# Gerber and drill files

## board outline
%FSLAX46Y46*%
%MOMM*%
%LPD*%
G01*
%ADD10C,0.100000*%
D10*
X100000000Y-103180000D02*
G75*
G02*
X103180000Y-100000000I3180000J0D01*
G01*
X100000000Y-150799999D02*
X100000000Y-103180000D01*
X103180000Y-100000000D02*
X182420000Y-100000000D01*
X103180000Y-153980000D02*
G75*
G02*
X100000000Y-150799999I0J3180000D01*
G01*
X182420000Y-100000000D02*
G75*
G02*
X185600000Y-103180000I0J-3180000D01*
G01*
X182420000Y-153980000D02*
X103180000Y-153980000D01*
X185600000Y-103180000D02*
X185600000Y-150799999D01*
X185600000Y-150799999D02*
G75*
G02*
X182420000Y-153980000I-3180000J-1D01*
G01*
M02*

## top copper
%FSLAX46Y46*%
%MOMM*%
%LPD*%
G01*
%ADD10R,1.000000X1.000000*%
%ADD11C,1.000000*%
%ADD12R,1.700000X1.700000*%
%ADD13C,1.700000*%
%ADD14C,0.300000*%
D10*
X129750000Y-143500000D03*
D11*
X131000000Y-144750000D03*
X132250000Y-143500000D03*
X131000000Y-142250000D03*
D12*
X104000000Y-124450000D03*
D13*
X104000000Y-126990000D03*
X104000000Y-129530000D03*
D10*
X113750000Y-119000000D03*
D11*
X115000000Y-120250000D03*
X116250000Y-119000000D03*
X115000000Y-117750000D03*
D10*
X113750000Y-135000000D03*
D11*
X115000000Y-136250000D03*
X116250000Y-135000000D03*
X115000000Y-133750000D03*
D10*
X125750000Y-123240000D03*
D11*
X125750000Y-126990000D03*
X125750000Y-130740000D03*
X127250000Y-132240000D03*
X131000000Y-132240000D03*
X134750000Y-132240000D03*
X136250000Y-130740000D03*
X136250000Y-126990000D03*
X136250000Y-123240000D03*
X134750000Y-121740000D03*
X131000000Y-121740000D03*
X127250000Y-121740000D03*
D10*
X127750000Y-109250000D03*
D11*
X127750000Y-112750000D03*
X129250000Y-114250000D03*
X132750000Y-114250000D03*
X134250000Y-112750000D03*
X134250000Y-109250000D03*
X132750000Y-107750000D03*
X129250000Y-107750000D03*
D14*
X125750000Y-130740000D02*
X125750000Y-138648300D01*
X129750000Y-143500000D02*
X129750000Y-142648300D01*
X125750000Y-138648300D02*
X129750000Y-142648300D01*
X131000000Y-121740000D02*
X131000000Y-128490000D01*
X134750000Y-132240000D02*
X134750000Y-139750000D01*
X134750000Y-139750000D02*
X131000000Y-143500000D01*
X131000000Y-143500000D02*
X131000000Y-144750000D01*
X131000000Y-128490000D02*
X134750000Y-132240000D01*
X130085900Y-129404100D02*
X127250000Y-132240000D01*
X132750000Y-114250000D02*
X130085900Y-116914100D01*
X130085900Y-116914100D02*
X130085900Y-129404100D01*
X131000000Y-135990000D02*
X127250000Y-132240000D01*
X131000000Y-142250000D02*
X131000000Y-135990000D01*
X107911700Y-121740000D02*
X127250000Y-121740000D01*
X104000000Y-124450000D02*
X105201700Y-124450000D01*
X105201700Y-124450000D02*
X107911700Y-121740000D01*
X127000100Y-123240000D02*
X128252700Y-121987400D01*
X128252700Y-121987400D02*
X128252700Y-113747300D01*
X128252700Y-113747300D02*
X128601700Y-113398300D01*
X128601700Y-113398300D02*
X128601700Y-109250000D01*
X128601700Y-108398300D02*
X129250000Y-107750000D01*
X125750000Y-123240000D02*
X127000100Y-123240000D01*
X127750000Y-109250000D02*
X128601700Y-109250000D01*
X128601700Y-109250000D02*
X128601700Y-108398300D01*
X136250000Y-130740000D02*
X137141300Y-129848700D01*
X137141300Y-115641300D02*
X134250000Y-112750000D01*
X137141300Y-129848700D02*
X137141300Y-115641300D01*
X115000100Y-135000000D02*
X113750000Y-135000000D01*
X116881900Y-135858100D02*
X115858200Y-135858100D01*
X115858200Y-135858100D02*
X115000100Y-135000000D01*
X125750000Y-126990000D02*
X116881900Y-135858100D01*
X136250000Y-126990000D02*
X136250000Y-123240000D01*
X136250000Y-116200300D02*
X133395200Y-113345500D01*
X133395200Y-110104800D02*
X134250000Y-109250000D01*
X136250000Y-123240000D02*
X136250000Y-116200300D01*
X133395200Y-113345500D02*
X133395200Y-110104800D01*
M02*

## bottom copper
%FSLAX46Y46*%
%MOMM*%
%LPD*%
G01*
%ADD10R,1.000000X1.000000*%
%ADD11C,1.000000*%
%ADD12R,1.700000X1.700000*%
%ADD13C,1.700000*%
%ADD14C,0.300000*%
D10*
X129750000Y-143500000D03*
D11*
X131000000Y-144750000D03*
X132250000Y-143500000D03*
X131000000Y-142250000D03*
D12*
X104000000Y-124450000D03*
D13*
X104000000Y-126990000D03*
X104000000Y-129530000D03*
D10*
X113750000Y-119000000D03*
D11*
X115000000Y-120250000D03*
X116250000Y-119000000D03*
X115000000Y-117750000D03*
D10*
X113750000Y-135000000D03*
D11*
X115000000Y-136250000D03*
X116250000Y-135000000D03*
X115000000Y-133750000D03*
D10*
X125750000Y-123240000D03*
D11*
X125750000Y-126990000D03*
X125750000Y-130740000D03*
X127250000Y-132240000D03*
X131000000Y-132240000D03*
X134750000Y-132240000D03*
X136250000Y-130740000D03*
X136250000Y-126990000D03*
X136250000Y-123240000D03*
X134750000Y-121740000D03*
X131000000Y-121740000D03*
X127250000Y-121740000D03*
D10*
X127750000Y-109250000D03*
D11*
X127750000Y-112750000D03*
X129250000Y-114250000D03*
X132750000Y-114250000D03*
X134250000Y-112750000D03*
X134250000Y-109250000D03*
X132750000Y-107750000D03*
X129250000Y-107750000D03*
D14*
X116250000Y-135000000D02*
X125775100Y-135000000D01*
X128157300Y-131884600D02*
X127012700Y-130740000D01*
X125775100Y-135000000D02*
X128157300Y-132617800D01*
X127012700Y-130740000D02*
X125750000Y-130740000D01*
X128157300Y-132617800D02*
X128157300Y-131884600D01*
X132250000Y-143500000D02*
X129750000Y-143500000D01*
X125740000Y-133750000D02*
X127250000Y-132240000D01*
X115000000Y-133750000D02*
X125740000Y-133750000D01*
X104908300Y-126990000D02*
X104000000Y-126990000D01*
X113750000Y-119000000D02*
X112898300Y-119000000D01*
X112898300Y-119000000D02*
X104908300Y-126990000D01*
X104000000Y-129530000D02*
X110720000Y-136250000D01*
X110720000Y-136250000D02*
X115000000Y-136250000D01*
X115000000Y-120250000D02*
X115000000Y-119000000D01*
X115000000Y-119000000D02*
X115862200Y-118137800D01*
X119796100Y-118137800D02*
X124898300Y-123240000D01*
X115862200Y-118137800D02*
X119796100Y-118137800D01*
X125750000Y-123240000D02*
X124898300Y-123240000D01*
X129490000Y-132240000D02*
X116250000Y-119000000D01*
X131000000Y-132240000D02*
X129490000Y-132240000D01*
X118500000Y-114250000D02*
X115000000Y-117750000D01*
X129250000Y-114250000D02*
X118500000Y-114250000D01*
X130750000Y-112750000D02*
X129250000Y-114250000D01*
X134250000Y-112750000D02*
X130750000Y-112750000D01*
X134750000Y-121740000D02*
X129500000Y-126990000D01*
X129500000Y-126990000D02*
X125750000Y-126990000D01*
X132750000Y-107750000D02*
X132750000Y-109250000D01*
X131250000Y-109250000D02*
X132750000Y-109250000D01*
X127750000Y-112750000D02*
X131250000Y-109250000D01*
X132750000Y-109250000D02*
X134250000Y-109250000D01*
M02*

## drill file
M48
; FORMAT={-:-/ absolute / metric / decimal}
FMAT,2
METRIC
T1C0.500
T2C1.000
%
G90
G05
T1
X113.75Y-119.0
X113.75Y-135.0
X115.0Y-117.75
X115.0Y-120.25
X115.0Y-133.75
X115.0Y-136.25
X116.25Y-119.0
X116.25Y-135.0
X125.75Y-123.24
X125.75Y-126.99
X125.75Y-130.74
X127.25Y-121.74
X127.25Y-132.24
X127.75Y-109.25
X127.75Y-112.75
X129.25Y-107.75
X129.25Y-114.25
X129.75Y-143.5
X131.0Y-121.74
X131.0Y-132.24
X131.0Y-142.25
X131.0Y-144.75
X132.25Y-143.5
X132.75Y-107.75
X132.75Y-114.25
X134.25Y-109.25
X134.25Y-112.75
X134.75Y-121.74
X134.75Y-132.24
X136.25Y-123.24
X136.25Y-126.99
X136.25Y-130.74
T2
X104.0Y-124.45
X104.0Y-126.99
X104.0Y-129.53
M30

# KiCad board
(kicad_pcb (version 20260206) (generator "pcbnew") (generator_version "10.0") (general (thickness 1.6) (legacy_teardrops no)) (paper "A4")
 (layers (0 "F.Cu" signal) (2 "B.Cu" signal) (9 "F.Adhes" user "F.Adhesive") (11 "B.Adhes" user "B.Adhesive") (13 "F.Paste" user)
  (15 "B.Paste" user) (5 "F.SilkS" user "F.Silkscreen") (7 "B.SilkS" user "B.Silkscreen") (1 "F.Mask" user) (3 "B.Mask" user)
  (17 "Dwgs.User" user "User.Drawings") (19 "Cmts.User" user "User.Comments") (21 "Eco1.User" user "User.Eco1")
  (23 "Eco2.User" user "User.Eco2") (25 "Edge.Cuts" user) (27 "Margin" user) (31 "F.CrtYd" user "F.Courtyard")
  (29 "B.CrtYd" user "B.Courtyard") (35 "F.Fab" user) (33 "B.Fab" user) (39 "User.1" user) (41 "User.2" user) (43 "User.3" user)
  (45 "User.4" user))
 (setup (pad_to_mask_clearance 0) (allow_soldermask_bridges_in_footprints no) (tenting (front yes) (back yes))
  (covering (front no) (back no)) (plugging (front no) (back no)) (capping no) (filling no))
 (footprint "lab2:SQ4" (layer "F.Cu") (at 131 143.5)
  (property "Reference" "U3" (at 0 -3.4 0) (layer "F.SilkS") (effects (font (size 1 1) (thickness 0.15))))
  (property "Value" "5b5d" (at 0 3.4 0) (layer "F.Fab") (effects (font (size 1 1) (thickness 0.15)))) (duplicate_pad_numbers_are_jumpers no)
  (pad "1" thru_hole rect (at -1.25 0) (size 1 1) (drill 0.5) (layers "*.Cu" "*.Mask") (remove_unused_layers no) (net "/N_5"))
  (pad "2" thru_hole circle (at 0 1.25) (size 1 1) (drill 0.5) (layers "*.Cu" "*.Mask") (remove_unused_layers no) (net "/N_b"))
  (pad "3" thru_hole circle (at 1.25 0) (size 1 1) (drill 0.5) (layers "*.Cu" "*.Mask") (remove_unused_layers no) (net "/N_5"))
  (pad "4" thru_hole circle (at 0 -1.25) (size 1 1) (drill 0.5) (layers "*.Cu" "*.Mask") (remove_unused_layers no) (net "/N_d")))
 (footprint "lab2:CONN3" (layer "F.Cu") (at 104 126.99)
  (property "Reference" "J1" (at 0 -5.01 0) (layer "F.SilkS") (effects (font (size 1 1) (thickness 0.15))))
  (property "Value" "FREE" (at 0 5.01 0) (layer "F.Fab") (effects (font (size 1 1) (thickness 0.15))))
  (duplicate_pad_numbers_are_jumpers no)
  (pad "1" thru_hole rect (at 0 -2.54) (size 1.7 1.7) (drill 1) (layers "*.Cu" "*.Mask") (remove_unused_layers no) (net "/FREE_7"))
  (pad "2" thru_hole circle (at 0 0) (size 1.7 1.7) (drill 1) (layers "*.Cu" "*.Mask") (remove_unused_layers no) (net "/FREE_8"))
  (pad "3" thru_hole circle (at 0 2.54) (size 1.7 1.7) (drill 1) (layers "*.Cu" "*.Mask") (remove_unused_layers no) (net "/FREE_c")))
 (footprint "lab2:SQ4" (layer "F.Cu") (at 115 119)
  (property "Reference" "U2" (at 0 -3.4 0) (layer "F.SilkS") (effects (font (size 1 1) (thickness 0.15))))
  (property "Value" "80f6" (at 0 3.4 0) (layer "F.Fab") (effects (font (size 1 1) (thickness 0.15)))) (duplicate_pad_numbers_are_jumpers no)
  (pad "1" thru_hole rect (at -1.25 0) (size 1 1) (drill 0.5) (layers "*.Cu" "*.Mask") (remove_unused_layers no) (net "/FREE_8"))
  (pad "2" thru_hole circle (at 0 1.25) (size 1 1) (drill 0.5) (layers "*.Cu" "*.Mask") (remove_unused_layers no) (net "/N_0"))
  (pad "3" thru_hole circle (at 1.25 0) (size 1 1) (drill 0.5) (layers "*.Cu" "*.Mask") (remove_unused_layers no) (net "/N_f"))
  (pad "4" thru_hole circle (at 0 -1.25) (size 1 1) (drill 0.5) (layers "*.Cu" "*.Mask") (remove_unused_layers no) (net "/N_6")))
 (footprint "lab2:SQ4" (layer "F.Cu") (at 115 135)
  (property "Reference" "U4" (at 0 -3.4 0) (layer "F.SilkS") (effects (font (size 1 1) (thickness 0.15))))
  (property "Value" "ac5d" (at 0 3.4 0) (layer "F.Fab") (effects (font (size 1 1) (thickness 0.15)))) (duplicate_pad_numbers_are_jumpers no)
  (pad "1" thru_hole rect (at -1.25 0) (size 1 1) (drill 0.5) (layers "*.Cu" "*.Mask") (remove_unused_layers no) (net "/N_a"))
  (pad "2" thru_hole circle (at 0 1.25) (size 1 1) (drill 0.5) (layers "*.Cu" "*.Mask") (remove_unused_layers no) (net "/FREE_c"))
  (pad "3" thru_hole circle (at 1.25 0) (size 1 1) (drill 0.5) (layers "*.Cu" "*.Mask") (remove_unused_layers no) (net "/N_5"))
  (pad "4" thru_hole circle (at 0 -1.25) (size 1 1) (drill 0.5) (layers "*.Cu" "*.Mask") (remove_unused_layers no) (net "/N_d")))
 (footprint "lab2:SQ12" (layer "F.Cu") (at 131 126.99)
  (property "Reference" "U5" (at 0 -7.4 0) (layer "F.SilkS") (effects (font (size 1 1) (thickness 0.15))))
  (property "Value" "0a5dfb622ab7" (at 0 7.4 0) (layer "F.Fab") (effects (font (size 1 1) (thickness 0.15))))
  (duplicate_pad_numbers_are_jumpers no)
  (pad "1" thru_hole rect (at -5.25 -3.75) (size 1 1) (drill 0.5) (layers "*.Cu" "*.Mask") (remove_unused_layers no) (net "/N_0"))
  (pad "2" thru_hole circle (at -5.25 0) (size 1 1) (drill 0.5) (layers "*.Cu" "*.Mask") (remove_unused_layers no) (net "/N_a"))
  (pad "3" thru_hole circle (at -5.25 3.75) (size 1 1) (drill 0.5) (layers "*.Cu" "*.Mask") (remove_unused_layers no) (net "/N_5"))
  (pad "4" thru_hole circle (at -3.75 5.25) (size 1 1) (drill 0.5) (layers "*.Cu" "*.Mask") (remove_unused_layers no) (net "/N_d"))
  (pad "5" thru_hole circle (at 0 5.25) (size 1 1) (drill 0.5) (layers "*.Cu" "*.Mask") (remove_unused_layers no) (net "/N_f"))
  (pad "6" thru_hole circle (at 3.75 5.25) (size 1 1) (drill 0.5) (layers "*.Cu" "*.Mask") (remove_unused_layers no) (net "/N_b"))
  (pad "7" thru_hole circle (at 5.25 3.75) (size 1 1) (drill 0.5) (layers "*.Cu" "*.Mask") (remove_unused_layers no) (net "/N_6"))
  (pad "8" thru_hole circle (at 5.25 0) (size 1 1) (drill 0.5) (layers "*.Cu" "*.Mask") (remove_unused_layers no) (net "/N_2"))
  (pad "9" thru_hole circle (at 5.25 -3.75) (size 1 1) (drill 0.5) (layers "*.Cu" "*.Mask") (remove_unused_layers no) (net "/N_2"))
  (pad "10" thru_hole circle (at 3.75 -5.25) (size 1 1) (drill 0.5) (layers "*.Cu" "*.Mask") (remove_unused_layers no) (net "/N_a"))
  (pad "11" thru_hole circle (at 0 -5.25) (size 1 1) (drill 0.5) (layers "*.Cu" "*.Mask") (remove_unused_layers no) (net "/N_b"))
  (pad "12" thru_hole circle (at -3.75 -5.25) (size 1 1) (drill 0.5) (layers "*.Cu" "*.Mask") (remove_unused_layers no) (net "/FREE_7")))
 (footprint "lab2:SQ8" (layer "F.Cu") (at 131 111)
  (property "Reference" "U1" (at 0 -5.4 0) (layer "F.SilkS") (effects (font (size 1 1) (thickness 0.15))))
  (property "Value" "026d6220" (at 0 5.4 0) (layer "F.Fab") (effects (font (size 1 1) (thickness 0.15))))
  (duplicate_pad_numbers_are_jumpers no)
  (pad "1" thru_hole rect (at -3.25 -1.75) (size 1 1) (drill 0.5) (layers "*.Cu" "*.Mask") (remove_unused_layers no) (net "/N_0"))
  (pad "2" thru_hole circle (at -3.25 1.75) (size 1 1) (drill 0.5) (layers "*.Cu" "*.Mask") (remove_unused_layers no) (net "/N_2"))
  (pad "3" thru_hole circle (at -1.75 3.25) (size 1 1) (drill 0.5) (layers "*.Cu" "*.Mask") (remove_unused_layers no) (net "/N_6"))
  (pad "4" thru_hole circle (at 1.75 3.25) (size 1 1) (drill 0.5) (layers "*.Cu" "*.Mask") (remove_unused_layers no) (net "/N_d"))
  (pad "5" thru_hole circle (at 3.25 1.75) (size 1 1) (drill 0.5) (layers "*.Cu" "*.Mask") (remove_unused_layers no) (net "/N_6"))
  (pad "6" thru_hole circle (at 3.25 -1.75) (size 1 1) (drill 0.5) (layers "*.Cu" "*.Mask") (remove_unused_layers no) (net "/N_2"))
  (pad "7" thru_hole circle (at 1.75 -3.25) (size 1 1) (drill 0.5) (layers "*.Cu" "*.Mask") (remove_unused_layers no) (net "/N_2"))
  (pad "8" thru_hole circle (at -1.75 -3.25) (size 1 1) (drill 0.5) (layers "*.Cu" "*.Mask") (remove_unused_layers no) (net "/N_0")))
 (gr_arc (start 100 103.18) (mid 100.9314 100.9314) (end 103.18 100) (stroke (width 0.1) (type default)) (layer "Edge.Cuts"))
 (gr_line (start 100 150.799999) (end 100 103.18) (stroke (width 0.1) (type default)) (layer "Edge.Cuts"))
 (gr_line (start 103.18 100) (end 182.42 100) (stroke (width 0.1) (type default)) (layer "Edge.Cuts"))
 (gr_arc (start 103.18 153.98) (mid 100.9314 153.048599) (end 100 150.799999) (stroke (width 0.1) (type default)) (layer "Edge.Cuts"))
 (gr_arc (start 182.42 100) (mid 184.668599 100.9314) (end 185.6 103.18) (stroke (width 0.1) (type default)) (layer "Edge.Cuts"))
 (gr_line (start 182.42 153.98) (end 103.18 153.98) (stroke (width 0.1) (type default)) (layer "Edge.Cuts"))
 (gr_line (start 185.6 103.18) (end 185.6 150.799999) (stroke (width 0.1) (type default)) (layer "Edge.Cuts"))
 (gr_arc (start 185.6 150.799999) (mid 184.668599 153.048599) (end 182.42 153.98) (stroke (width 0.1) (type default)) (layer "Edge.Cuts"))
 (segment (start 125.75 130.74) (end 125.75 138.6483) (width 0.3) (layer "F.Cu") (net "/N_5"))
 (segment (start 129.75 143.5) (end 129.75 142.6483) (width 0.3) (layer "F.Cu") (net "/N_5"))
 (segment (start 125.75 138.6483) (end 129.75 142.6483) (width 0.3) (layer "F.Cu") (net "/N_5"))
 (segment (start 116.25 135) (end 125.7751 135) (width 0.3) (layer "B.Cu") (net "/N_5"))
 (segment (start 128.1573 131.8846) (end 127.0127 130.74) (width 0.3) (layer "B.Cu") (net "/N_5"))
 (segment (start 125.7751 135) (end 128.1573 132.6178) (width 0.3) (layer "B.Cu") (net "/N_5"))
 (segment (start 127.0127 130.74) (end 125.75 130.74) (width 0.3) (layer "B.Cu") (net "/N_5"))
 (segment (start 128.1573 132.6178) (end 128.1573 131.8846) (width 0.3) (layer "B.Cu") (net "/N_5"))
 (segment (start 132.25 143.5) (end 129.75 143.5) (width 0.3) (layer "B.Cu") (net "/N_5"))
 (segment (start 131 121.74) (end 131 128.49) (width 0.3) (layer "F.Cu") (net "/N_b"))
 (segment (start 134.75 132.24) (end 134.75 139.75) (width 0.3) (layer "F.Cu") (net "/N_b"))
 (segment (start 134.75 139.75) (end 131 143.5) (width 0.3) (layer "F.Cu") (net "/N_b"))
 (segment (start 131 143.5) (end 131 144.75) (width 0.3) (layer "F.Cu") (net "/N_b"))
 (segment (start 131 128.49) (end 134.75 132.24) (width 0.3) (layer "F.Cu") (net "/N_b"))
 (segment (start 130.0859 129.4041) (end 127.25 132.24) (width 0.3) (layer "F.Cu") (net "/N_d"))
 (segment (start 132.75 114.25) (end 130.0859 116.9141) (width 0.3) (layer "F.Cu") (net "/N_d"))
 (segment (start 130.0859 116.9141) (end 130.0859 129.4041) (width 0.3) (layer "F.Cu") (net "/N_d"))
 (segment (start 131 135.99) (end 127.25 132.24) (width 0.3) (layer "F.Cu") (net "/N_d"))
 (segment (start 131 142.25) (end 131 135.99) (width 0.3) (layer "F.Cu") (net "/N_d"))
 (segment (start 125.74 133.75) (end 127.25 132.24) (width 0.3) (layer "B.Cu") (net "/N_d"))
 (segment (start 115 133.75) (end 125.74 133.75) (width 0.3) (layer "B.Cu") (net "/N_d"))
 (segment (start 107.9117 121.74) (end 127.25 121.74) (width 0.3) (layer "F.Cu") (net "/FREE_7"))
 (segment (start 104 124.45) (end 105.2017 124.45) (width 0.3) (layer "F.Cu") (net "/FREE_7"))
 (segment (start 105.2017 124.45) (end 107.9117 121.74) (width 0.3) (layer "F.Cu") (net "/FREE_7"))
 (segment (start 104.9083 126.99) (end 104 126.99) (width 0.3) (layer "B.Cu") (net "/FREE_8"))
 (segment (start 113.75 119) (end 112.8983 119) (width 0.3) (layer "B.Cu") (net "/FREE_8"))
 (segment (start 112.8983 119) (end 104.9083 126.99) (width 0.3) (layer "B.Cu") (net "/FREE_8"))
 (segment (start 104 129.53) (end 110.72 136.25) (width 0.3) (layer "B.Cu") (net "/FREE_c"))
 (segment (start 110.72 136.25) (end 115 136.25) (width 0.3) (layer "B.Cu") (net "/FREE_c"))
 (segment (start 127.0001 123.24) (end 128.2527 121.9874) (width 0.3) (layer "F.Cu") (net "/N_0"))
 (segment (start 128.2527 121.9874) (end 128.2527 113.7473) (width 0.3) (layer "F.Cu") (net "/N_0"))
 (segment (start 128.2527 113.7473) (end 128.6017 113.3983) (width 0.3) (layer "F.Cu") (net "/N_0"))
 (segment (start 128.6017 113.3983) (end 128.6017 109.25) (width 0.3) (layer "F.Cu") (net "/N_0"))
 (segment (start 128.6017 108.3983) (end 129.25 107.75) (width 0.3) (layer "F.Cu") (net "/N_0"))
 (segment (start 125.75 123.24) (end 127.0001 123.24) (width 0.3) (layer "F.Cu") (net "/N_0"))
 (segment (start 127.75 109.25) (end 128.6017 109.25) (width 0.3) (layer "F.Cu") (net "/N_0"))
 (segment (start 128.6017 109.25) (end 128.6017 108.3983) (width 0.3) (layer "F.Cu") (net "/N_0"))
 (segment (start 115 120.25) (end 115 119) (width 0.3) (layer "B.Cu") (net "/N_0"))
 (segment (start 115 119) (end 115.8622 118.1378) (width 0.3) (layer "B.Cu") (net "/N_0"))
 (segment (start 119.7961 118.1378) (end 124.8983 123.24) (width 0.3) (layer "B.Cu") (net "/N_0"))
 (segment (start 115.8622 118.1378) (end 119.7961 118.1378) (width 0.3) (layer "B.Cu") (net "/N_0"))
 (segment (start 125.75 123.24) (end 124.8983 123.24) (width 0.3) (layer "B.Cu") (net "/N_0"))
 (segment (start 129.49 132.24) (end 116.25 119) (width 0.3) (layer "B.Cu") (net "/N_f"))
 (segment (start 131 132.24) (end 129.49 132.24) (width 0.3) (layer "B.Cu") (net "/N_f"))
 (segment (start 136.25 130.74) (end 137.1413 129.8487) (width 0.3) (layer "F.Cu") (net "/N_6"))
 (segment (start 137.1413 115.6413) (end 134.25 112.75) (width 0.3) (layer "F.Cu") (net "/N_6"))
 (segment (start 137.1413 129.8487) (end 137.1413 115.6413) (width 0.3) (layer "F.Cu") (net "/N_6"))
 (segment (start 118.5 114.25) (end 115 117.75) (width 0.3) (layer "B.Cu") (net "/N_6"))
 (segment (start 129.25 114.25) (end 118.5 114.25) (width 0.3) (layer "B.Cu") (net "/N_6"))
 (segment (start 130.75 112.75) (end 129.25 114.25) (width 0.3) (layer "B.Cu") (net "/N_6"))
 (segment (start 134.25 112.75) (end 130.75 112.75) (width 0.3) (layer "B.Cu") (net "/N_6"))
 (segment (start 115.0001 135) (end 113.75 135) (width 0.3) (layer "F.Cu") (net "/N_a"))
 (segment (start 116.8819 135.8581) (end 115.8582 135.8581) (width 0.3) (layer "F.Cu") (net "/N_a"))
 (segment (start 115.8582 135.8581) (end 115.0001 135) (width 0.3) (layer "F.Cu") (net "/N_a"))
 (segment (start 125.75 126.99) (end 116.8819 135.8581) (width 0.3) (layer "F.Cu") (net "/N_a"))
 (segment (start 134.75 121.74) (end 129.5 126.99) (width 0.3) (layer "B.Cu") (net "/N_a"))
 (segment (start 129.5 126.99) (end 125.75 126.99) (width 0.3) (layer "B.Cu") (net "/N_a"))
 (segment (start 136.25 126.99) (end 136.25 123.24) (width 0.3) (layer "F.Cu") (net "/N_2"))
 (segment (start 136.25 116.2003) (end 133.3952 113.3455) (width 0.3) (layer "F.Cu") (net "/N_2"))
 (segment (start 133.3952 110.1048) (end 134.25 109.25) (width 0.3) (layer "F.Cu") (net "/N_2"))
 (segment (start 136.25 123.24) (end 136.25 116.2003) (width 0.3) (layer "F.Cu") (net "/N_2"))
 (segment (start 133.3952 113.3455) (end 133.3952 110.1048) (width 0.3) (layer "F.Cu") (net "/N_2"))
 (segment (start 132.75 107.75) (end 132.75 109.25) (width 0.3) (layer "B.Cu") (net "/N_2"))
 (segment (start 131.25 109.25) (end 132.75 109.25) (width 0.3) (layer "B.Cu") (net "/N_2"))
 (segment (start 127.75 112.75) (end 131.25 109.25) (width 0.3) (layer "B.Cu") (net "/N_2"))
 (segment (start 132.75 109.25) (end 134.25 109.25) (width 0.3) (layer "B.Cu") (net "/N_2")))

